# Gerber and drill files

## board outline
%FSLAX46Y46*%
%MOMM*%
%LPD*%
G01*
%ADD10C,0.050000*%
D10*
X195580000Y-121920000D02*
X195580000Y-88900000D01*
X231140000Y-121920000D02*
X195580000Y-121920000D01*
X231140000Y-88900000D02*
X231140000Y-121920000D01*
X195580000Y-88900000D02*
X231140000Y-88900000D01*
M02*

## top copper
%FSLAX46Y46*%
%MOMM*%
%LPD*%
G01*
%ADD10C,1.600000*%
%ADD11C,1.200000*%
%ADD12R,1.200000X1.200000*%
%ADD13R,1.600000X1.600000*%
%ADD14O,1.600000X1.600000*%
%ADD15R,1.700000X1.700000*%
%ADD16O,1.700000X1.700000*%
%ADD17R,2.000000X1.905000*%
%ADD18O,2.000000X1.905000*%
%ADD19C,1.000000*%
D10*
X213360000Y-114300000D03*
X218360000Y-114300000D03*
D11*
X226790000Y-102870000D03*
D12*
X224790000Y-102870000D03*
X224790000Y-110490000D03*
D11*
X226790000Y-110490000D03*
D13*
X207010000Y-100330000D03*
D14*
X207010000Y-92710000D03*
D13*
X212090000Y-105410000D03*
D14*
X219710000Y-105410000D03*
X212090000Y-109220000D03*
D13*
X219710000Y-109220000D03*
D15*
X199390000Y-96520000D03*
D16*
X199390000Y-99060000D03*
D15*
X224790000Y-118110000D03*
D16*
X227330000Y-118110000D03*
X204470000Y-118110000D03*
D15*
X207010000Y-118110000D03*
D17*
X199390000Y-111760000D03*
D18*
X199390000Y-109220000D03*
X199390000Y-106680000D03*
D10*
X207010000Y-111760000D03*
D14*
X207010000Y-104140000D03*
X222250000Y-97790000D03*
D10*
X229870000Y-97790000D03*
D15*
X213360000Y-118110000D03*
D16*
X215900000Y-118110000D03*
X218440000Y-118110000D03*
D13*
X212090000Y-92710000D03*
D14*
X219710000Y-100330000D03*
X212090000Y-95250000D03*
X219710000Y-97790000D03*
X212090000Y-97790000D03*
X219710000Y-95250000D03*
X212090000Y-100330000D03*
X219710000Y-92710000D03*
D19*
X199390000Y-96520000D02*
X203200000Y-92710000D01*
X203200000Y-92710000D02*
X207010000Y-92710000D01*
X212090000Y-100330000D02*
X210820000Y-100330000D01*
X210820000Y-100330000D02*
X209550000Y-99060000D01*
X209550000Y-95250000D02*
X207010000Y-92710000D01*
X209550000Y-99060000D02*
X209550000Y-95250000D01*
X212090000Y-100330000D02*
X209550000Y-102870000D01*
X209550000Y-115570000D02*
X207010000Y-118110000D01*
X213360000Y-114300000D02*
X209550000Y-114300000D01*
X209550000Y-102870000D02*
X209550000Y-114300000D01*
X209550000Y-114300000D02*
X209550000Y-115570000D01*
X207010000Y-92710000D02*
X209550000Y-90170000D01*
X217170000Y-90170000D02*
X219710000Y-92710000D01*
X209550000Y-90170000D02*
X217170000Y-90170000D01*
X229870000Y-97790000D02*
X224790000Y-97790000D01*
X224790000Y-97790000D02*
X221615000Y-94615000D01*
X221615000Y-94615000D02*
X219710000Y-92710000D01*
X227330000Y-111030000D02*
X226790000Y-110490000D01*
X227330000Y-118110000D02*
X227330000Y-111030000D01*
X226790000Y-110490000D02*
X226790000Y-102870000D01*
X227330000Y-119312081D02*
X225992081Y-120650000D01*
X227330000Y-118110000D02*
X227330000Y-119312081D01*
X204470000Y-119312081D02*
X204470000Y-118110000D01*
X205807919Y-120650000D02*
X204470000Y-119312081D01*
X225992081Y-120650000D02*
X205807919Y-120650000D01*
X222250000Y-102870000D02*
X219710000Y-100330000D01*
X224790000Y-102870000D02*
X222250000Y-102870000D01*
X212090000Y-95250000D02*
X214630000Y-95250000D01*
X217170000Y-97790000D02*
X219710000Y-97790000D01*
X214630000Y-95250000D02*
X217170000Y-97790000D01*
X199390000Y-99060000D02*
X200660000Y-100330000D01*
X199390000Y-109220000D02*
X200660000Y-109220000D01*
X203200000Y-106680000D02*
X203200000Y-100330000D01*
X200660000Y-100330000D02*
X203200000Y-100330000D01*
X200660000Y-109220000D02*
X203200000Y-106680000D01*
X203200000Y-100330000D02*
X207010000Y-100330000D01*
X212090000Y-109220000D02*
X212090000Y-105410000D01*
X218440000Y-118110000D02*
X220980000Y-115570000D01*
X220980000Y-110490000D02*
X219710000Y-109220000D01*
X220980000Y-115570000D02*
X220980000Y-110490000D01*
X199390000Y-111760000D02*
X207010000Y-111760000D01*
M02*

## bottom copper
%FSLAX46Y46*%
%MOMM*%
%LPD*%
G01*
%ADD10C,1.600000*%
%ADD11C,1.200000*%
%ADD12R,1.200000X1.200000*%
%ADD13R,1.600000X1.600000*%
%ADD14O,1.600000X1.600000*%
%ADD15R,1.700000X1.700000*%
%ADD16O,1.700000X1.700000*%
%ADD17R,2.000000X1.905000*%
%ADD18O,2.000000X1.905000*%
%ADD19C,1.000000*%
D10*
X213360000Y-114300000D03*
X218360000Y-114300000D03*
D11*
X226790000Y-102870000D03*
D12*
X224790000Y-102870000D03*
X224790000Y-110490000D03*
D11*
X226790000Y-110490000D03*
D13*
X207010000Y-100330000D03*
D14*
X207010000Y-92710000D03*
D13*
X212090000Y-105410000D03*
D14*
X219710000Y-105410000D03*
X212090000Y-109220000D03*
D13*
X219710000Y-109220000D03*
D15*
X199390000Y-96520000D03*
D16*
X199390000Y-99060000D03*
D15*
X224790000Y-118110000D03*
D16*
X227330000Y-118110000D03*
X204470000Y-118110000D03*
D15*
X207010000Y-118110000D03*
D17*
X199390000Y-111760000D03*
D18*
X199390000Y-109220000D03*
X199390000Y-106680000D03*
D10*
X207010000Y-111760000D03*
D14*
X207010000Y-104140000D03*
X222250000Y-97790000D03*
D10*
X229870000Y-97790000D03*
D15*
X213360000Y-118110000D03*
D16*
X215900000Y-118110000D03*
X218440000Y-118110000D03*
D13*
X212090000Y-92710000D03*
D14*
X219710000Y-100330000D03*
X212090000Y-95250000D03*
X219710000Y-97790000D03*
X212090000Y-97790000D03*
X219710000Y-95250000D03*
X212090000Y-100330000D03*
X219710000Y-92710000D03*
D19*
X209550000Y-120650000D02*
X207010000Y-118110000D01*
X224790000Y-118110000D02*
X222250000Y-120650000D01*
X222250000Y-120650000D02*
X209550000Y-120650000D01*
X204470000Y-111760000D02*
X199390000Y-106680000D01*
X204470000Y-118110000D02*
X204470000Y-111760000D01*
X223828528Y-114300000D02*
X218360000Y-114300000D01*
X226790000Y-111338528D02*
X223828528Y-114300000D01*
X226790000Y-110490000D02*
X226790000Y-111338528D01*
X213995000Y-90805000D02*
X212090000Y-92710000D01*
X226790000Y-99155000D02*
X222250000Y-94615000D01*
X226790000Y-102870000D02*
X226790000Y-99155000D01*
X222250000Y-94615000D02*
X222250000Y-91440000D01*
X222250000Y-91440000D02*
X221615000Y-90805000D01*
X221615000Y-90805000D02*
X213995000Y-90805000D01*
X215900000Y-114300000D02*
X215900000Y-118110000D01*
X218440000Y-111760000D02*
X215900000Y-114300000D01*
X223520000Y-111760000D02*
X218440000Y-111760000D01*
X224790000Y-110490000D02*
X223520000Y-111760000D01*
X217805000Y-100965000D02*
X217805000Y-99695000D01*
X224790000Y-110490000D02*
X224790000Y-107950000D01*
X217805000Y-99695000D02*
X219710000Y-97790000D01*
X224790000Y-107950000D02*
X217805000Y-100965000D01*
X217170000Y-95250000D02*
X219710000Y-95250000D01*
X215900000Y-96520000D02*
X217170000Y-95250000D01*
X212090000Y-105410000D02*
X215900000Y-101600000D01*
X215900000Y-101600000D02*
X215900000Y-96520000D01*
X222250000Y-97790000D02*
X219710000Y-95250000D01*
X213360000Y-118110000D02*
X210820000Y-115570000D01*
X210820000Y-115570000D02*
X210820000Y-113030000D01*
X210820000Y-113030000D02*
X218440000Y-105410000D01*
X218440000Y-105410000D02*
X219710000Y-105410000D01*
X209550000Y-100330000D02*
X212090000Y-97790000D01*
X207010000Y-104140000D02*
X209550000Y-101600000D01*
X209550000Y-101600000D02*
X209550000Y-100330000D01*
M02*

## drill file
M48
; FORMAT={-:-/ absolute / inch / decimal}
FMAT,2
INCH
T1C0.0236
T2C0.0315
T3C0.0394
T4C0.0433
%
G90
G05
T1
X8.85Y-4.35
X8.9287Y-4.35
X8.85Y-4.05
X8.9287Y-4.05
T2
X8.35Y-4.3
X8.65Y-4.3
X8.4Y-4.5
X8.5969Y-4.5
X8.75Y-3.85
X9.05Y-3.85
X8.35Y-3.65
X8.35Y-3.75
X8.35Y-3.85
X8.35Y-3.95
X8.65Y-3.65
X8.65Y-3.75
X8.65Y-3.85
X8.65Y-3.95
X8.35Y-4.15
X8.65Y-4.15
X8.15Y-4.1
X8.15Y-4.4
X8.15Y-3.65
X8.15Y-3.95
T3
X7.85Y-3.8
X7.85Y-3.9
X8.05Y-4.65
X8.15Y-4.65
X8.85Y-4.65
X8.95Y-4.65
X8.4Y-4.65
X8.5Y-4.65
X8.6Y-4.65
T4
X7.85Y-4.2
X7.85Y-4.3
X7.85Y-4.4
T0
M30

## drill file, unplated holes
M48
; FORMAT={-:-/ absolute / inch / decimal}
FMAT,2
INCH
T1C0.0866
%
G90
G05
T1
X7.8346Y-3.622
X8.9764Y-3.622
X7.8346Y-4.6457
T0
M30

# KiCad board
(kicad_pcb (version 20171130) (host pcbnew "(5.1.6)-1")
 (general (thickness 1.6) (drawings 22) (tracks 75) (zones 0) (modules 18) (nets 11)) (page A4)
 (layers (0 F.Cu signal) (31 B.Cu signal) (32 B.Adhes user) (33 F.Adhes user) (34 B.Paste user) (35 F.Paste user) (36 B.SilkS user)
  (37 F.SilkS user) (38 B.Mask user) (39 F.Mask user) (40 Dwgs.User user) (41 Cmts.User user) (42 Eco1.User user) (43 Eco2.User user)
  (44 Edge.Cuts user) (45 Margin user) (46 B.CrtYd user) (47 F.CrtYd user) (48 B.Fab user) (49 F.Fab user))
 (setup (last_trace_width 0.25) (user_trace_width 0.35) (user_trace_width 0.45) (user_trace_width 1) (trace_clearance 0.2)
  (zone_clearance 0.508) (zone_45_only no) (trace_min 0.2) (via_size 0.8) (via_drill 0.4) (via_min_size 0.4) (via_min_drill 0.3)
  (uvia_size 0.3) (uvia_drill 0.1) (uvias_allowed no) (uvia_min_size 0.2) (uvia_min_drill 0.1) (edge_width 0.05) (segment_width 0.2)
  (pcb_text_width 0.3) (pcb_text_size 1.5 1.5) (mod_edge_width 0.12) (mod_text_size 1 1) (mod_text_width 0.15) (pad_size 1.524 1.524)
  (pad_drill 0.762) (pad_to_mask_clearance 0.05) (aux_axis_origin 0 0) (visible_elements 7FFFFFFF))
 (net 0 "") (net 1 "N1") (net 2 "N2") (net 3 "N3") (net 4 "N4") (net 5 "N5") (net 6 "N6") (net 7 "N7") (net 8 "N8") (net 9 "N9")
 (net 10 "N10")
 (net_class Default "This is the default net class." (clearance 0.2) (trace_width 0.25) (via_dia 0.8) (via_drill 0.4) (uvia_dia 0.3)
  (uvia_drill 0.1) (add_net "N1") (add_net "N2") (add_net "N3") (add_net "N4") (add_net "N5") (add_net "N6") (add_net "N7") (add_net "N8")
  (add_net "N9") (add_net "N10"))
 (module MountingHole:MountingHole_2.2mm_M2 (layer F.Cu) (at 199 118)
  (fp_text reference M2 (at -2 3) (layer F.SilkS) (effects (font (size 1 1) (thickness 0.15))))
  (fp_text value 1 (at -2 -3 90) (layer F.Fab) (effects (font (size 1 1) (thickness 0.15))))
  (pad 1 np_thru_hole circle (at 0 0) (size 2.2 2.2) (drill 2.2) (layers *.Cu *.Mask)))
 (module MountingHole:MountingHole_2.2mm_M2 (layer F.Cu) (at 228 92)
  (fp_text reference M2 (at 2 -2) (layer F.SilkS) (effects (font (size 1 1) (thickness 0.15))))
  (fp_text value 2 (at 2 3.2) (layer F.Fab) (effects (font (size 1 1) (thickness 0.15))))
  (pad 1 np_thru_hole circle (at 0 0) (size 2.2 2.2) (drill 2.2) (layers *.Cu *.Mask)))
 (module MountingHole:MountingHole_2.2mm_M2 (layer F.Cu) (at 199 92)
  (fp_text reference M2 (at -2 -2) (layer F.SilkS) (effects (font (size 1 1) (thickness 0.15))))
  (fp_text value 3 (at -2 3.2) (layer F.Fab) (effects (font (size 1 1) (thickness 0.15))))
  (pad 1 np_thru_hole circle (at 0 0) (size 2.2 2.2) (drill 2.2) (layers *.Cu *.Mask)))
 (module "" (layer F.Cu) (at 133.35 157.48)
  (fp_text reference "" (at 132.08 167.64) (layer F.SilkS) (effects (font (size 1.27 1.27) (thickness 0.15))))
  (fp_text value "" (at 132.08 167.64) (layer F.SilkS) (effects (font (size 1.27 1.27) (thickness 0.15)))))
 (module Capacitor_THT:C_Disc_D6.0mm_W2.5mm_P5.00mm (layer F.Cu) (at 213.36 114.3)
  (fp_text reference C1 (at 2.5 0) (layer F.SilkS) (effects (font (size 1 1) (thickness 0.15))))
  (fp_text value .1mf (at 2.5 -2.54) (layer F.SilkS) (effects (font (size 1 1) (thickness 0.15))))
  (pad 1 thru_hole circle (at 0 0) (size 1.6 1.6) (drill 0.8) (layers *.Cu *.Mask) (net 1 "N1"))
  (pad 2 thru_hole circle (at 5 0) (size 1.6 1.6) (drill 0.8) (layers *.Cu *.Mask) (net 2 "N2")))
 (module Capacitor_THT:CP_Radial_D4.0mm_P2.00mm (layer F.Cu) (at 224.79 102.87)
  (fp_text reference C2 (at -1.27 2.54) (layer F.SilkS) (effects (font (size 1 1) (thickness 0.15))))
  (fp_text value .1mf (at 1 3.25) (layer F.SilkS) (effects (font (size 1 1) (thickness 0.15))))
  (pad 2 thru_hole circle (at 2 0) (size 1.2 1.2) (drill 0.6) (layers *.Cu *.Mask) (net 2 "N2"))
  (pad 1 thru_hole rect (at 0 0) (size 1.2 1.2) (drill 0.6) (layers *.Cu *.Mask) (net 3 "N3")))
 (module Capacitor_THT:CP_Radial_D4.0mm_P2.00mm (layer F.Cu) (at 224.79 110.49)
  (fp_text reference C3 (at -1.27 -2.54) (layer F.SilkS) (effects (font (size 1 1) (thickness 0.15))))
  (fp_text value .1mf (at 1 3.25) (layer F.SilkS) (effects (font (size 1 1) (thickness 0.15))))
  (pad 1 thru_hole rect (at 0 0) (size 1.2 1.2) (drill 0.6) (layers *.Cu *.Mask) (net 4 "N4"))
  (pad 2 thru_hole circle (at 2 0) (size 1.2 1.2) (drill 0.6) (layers *.Cu *.Mask) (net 2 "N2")))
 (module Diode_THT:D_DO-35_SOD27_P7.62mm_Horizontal (layer F.Cu) (at 207.01 100.33 90)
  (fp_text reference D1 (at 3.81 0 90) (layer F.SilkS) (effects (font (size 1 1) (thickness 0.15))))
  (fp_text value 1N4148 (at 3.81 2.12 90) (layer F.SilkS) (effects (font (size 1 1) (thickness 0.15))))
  (pad 1 thru_hole rect (at 0 0 90) (size 1.6 1.6) (drill 0.8) (layers *.Cu *.Mask) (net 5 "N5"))
  (pad 2 thru_hole oval (at 7.62 0 90) (size 1.6 1.6) (drill 0.8) (layers *.Cu *.Mask) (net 1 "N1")))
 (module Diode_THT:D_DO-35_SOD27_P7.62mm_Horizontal (layer F.Cu) (at 212.09 105.41)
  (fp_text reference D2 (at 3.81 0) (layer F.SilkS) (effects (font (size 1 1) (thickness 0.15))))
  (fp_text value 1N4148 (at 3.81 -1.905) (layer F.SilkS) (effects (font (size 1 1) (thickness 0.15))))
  (pad 1 thru_hole rect (at 0 0) (size 1.6 1.6) (drill 0.8) (layers *.Cu *.Mask) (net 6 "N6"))
  (pad 2 thru_hole oval (at 7.62 0) (size 1.6 1.6) (drill 0.8) (layers *.Cu *.Mask) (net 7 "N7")))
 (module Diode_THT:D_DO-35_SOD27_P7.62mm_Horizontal (layer F.Cu) (at 219.71 109.22 180)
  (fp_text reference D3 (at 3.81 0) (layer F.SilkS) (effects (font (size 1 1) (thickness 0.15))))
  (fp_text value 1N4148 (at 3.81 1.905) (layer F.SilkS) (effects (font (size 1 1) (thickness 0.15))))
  (pad 2 thru_hole oval (at 7.62 0 180) (size 1.6 1.6) (drill 0.8) (layers *.Cu *.Mask) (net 6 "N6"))
  (pad 1 thru_hole rect (at 0 0 180) (size 1.6 1.6) (drill 0.8) (layers *.Cu *.Mask) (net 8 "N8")))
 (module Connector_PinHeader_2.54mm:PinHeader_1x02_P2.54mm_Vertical (layer F.Cu) (at 199.39 96.52)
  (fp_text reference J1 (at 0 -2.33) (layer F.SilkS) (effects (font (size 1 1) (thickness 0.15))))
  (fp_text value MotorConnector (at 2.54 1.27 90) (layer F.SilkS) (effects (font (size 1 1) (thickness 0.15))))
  (pad 1 thru_hole rect (at 0 0) (size 1.7 1.7) (drill 1) (layers *.Cu *.Mask) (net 1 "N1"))
  (pad 2 thru_hole oval (at 0 2.54) (size 1.7 1.7) (drill 1) (layers *.Cu *.Mask) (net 5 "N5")))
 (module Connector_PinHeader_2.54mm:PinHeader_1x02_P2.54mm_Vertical (layer F.Cu) (at 224.79 118.11 90)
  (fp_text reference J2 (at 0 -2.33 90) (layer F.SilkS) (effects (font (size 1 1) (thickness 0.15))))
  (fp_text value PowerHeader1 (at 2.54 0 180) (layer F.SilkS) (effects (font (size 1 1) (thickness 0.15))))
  (pad 1 thru_hole rect (at 0 0 90) (size 1.7 1.7) (drill 1) (layers *.Cu *.Mask) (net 1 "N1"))
  (pad 2 thru_hole oval (at 0 2.54 90) (size 1.7 1.7) (drill 1) (layers *.Cu *.Mask) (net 2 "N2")))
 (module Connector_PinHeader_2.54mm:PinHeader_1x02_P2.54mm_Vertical (layer F.Cu) (at 207.01 118.11 270)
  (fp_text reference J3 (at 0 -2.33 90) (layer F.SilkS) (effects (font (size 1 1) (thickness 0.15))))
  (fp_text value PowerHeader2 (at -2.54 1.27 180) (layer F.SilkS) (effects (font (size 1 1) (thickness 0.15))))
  (pad 2 thru_hole oval (at 0 2.54 270) (size 1.7 1.7) (drill 1) (layers *.Cu *.Mask) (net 2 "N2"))
  (pad 1 thru_hole rect (at 0 0 270) (size 1.7 1.7) (drill 1) (layers *.Cu *.Mask) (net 1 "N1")))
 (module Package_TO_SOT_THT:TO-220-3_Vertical (layer F.Cu) (at 199.39 111.76 90)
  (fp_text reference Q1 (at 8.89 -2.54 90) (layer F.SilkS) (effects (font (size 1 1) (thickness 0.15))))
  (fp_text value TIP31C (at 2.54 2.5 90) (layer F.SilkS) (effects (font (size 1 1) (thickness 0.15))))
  (pad 1 thru_hole rect (at 0 0 90) (size 1.905 2) (drill 1.1) (layers *.Cu *.Mask) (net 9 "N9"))
  (pad 2 thru_hole oval (at 2.54 0 90) (size 1.905 2) (drill 1.1) (layers *.Cu *.Mask) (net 5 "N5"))
  (pad 3 thru_hole oval (at 5.08 0 90) (size 1.905 2) (drill 1.1) (layers *.Cu *.Mask) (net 2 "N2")))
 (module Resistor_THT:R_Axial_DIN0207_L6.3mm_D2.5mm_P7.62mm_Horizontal (layer F.Cu) (at 207.01 111.76 90)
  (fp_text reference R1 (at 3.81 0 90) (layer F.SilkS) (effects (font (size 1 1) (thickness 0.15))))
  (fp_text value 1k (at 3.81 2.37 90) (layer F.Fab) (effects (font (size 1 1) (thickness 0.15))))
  (pad 1 thru_hole circle (at 0 0 90) (size 1.6 1.6) (drill 0.8) (layers *.Cu *.Mask) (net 9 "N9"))
  (pad 2 thru_hole oval (at 7.62 0 90) (size 1.6 1.6) (drill 0.8) (layers *.Cu *.Mask) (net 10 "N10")))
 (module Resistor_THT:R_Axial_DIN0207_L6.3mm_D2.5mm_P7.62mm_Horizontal (layer F.Cu) (at 229.87 97.79 180)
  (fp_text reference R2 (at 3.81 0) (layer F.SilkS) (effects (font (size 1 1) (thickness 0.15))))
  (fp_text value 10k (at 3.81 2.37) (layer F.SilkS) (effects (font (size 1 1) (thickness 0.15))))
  (pad 2 thru_hole oval (at 7.62 0 180) (size 1.6 1.6) (drill 0.8) (layers *.Cu *.Mask) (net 6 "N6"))
  (pad 1 thru_hole circle (at 0 0 180) (size 1.6 1.6) (drill 0.8) (layers *.Cu *.Mask) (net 1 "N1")))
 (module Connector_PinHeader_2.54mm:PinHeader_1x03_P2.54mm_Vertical (layer F.Cu) (at 213.36 118.11 90)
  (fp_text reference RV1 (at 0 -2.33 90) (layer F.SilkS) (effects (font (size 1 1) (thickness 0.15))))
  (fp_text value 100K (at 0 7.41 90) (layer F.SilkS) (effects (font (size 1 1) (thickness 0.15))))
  (pad 1 thru_hole rect (at 0 0 90) (size 1.7 1.7) (drill 1) (layers *.Cu *.Mask) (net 7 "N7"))
  (pad 2 thru_hole oval (at 0 2.54 90) (size 1.7 1.7) (drill 1) (layers *.Cu *.Mask) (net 4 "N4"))
  (pad 3 thru_hole oval (at 0 5.08 90) (size 1.7 1.7) (drill 1) (layers *.Cu *.Mask) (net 8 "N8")))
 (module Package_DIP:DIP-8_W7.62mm (layer F.Cu) (at 212.09 92.71)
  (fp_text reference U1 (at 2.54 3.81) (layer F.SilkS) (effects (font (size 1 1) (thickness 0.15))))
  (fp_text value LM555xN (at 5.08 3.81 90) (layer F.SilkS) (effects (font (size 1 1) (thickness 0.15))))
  (pad 1 thru_hole rect (at 0 0) (size 1.6 1.6) (drill 0.8) (layers *.Cu *.Mask) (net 2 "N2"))
  (pad 5 thru_hole oval (at 7.62 7.62) (size 1.6 1.6) (drill 0.8) (layers *.Cu *.Mask) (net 3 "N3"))
  (pad 2 thru_hole oval (at 0 2.54) (size 1.6 1.6) (drill 0.8) (layers *.Cu *.Mask) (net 4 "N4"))
  (pad 6 thru_hole oval (at 7.62 5.08) (size 1.6 1.6) (drill 0.8) (layers *.Cu *.Mask) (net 4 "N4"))
  (pad 3 thru_hole oval (at 0 5.08) (size 1.6 1.6) (drill 0.8) (layers *.Cu *.Mask) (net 10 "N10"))
  (pad 7 thru_hole oval (at 7.62 2.54) (size 1.6 1.6) (drill 0.8) (layers *.Cu *.Mask) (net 6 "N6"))
  (pad 4 thru_hole oval (at 0 7.62) (size 1.6 1.6) (drill 0.8) (layers *.Cu *.Mask) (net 1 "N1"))
  (pad 8 thru_hole oval (at 7.62 0) (size 1.6 1.6) (drill 0.8) (layers *.Cu *.Mask) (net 1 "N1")))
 (gr_line (start 195.58 121.92) (end 195.58 88.9) (layer Edge.Cuts) (width 0.05))
 (gr_line (start 231.14 121.92) (end 195.58 121.92) (layer Edge.Cuts) (width 0.05))
 (gr_line (start 231.14 88.9) (end 231.14 121.92) (layer Edge.Cuts) (width 0.05))
 (gr_line (start 195.58 88.9) (end 231.14 88.9) (layer Edge.Cuts) (width 0.05))
 (segment (start 199.39 96.52) (end 203.2 92.71) (width 1) (layer F.Cu) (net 1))
 (segment (start 203.2 92.71) (end 207.01 92.71) (width 1) (layer F.Cu) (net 1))
 (segment (start 212.09 100.33) (end 210.82 100.33) (width 1) (layer F.Cu) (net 1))
 (segment (start 210.82 100.33) (end 209.55 99.06) (width 1) (layer F.Cu) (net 1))
 (segment (start 209.55 95.25) (end 207.01 92.71) (width 1) (layer F.Cu) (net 1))
 (segment (start 209.55 99.06) (end 209.55 95.25) (width 1) (layer F.Cu) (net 1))
 (segment (start 212.09 100.33) (end 209.55 102.87) (width 1) (layer F.Cu) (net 1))
 (segment (start 209.55 115.57) (end 207.01 118.11) (width 1) (layer F.Cu) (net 1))
 (segment (start 213.36 114.3) (end 209.55 114.3) (width 1) (layer F.Cu) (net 1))
 (segment (start 209.55 102.87) (end 209.55 114.3) (width 1) (layer F.Cu) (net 1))
 (segment (start 209.55 114.3) (end 209.55 115.57) (width 1) (layer F.Cu) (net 1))
 (segment (start 207.01 92.71) (end 209.55 90.17) (width 1) (layer F.Cu) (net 1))
 (segment (start 217.17 90.17) (end 219.71 92.71) (width 1) (layer F.Cu) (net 1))
 (segment (start 209.55 90.17) (end 217.17 90.17) (width 1) (layer F.Cu) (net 1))
 (segment (start 209.55 120.65) (end 207.01 118.11) (width 1) (layer B.Cu) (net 1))
 (segment (start 224.79 118.11) (end 222.25 120.65) (width 1) (layer B.Cu) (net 1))
 (segment (start 222.25 120.65) (end 209.55 120.65) (width 1) (layer B.Cu) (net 1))
 (segment (start 229.87 97.79) (end 224.79 97.79) (width 1) (layer F.Cu) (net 1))
 (segment (start 224.79 97.79) (end 221.615 94.615) (width 1) (layer F.Cu) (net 1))
 (segment (start 221.615 94.615) (end 219.71 92.71) (width 1) (layer F.Cu) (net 1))
 (segment (start 227.33 111.03) (end 226.79 110.49) (width 1) (layer F.Cu) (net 2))
 (segment (start 227.33 118.11) (end 227.33 111.03) (width 1) (layer F.Cu) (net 2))
 (segment (start 226.79 110.49) (end 226.79 102.87) (width 1) (layer F.Cu) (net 2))
 (segment (start 204.47 111.76) (end 199.39 106.68) (width 1) (layer B.Cu) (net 2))
 (segment (start 204.47 118.11) (end 204.47 111.76) (width 1) (layer B.Cu) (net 2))
 (segment (start 223.828528 114.3) (end 218.36 114.3) (width 1) (layer B.Cu) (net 2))
 (segment (start 226.79 111.338528) (end 223.828528 114.3) (width 1) (layer B.Cu) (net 2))
 (segment (start 226.79 110.49) (end 226.79 111.338528) (width 1) (layer B.Cu) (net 2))
 (segment (start 227.33 119.312081) (end 225.992081 120.65) (width 1) (layer F.Cu) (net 2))
 (segment (start 227.33 118.11) (end 227.33 119.312081) (width 1) (layer F.Cu) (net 2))
 (segment (start 204.47 119.312081) (end 204.47 118.11) (width 1) (layer F.Cu) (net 2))
 (segment (start 205.807919 120.65) (end 204.47 119.312081) (width 1) (layer F.Cu) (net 2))
 (segment (start 225.992081 120.65) (end 205.807919 120.65) (width 1) (layer F.Cu) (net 2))
 (segment (start 213.995 90.805) (end 212.09 92.71) (width 1) (layer B.Cu) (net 2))
 (segment (start 226.79 99.155) (end 222.25 94.615) (width 1) (layer B.Cu) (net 2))
 (segment (start 226.79 102.87) (end 226.79 99.155) (width 1) (layer B.Cu) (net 2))
 (segment (start 222.25 94.615) (end 222.25 91.44) (width 1) (layer B.Cu) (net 2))
 (segment (start 222.25 91.44) (end 221.615 90.805) (width 1) (layer B.Cu) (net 2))
 (segment (start 221.615 90.805) (end 213.995 90.805) (width 1) (layer B.Cu) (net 2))
 (segment (start 222.25 102.87) (end 219.71 100.33) (width 1) (layer F.Cu) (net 3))
 (segment (start 224.79 102.87) (end 222.25 102.87) (width 1) (layer F.Cu) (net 3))
 (segment (start 212.09 95.25) (end 214.63 95.25) (width 1) (layer F.Cu) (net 4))
 (segment (start 217.17 97.79) (end 219.71 97.79) (width 1) (layer F.Cu) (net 4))
 (segment (start 214.63 95.25) (end 217.17 97.79) (width 1) (layer F.Cu) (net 4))
 (segment (start 215.9 114.3) (end 215.9 118.11) (width 1) (layer B.Cu) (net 4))
 (segment (start 218.44 111.76) (end 215.9 114.3) (width 1) (layer B.Cu) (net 4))
 (segment (start 223.52 111.76) (end 218.44 111.76) (width 1) (layer B.Cu) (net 4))
 (segment (start 224.79 110.49) (end 223.52 111.76) (width 1) (layer B.Cu) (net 4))
 (segment (start 217.805 100.965) (end 217.805 99.695) (width 1) (layer B.Cu) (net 4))
 (segment (start 224.79 110.49) (end 224.79 107.95) (width 1) (layer B.Cu) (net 4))
 (segment (start 217.805 99.695) (end 219.71 97.79) (width 1) (layer B.Cu) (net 4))
 (segment (start 224.79 107.95) (end 217.805 100.965) (width 1) (layer B.Cu) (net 4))
 (segment (start 199.39 99.06) (end 200.66 100.33) (width 1) (layer F.Cu) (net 5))
 (segment (start 199.39 109.22) (end 200.66 109.22) (width 1) (layer F.Cu) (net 5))
 (segment (start 203.2 106.68) (end 203.2 100.33) (width 1) (layer F.Cu) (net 5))
 (segment (start 200.66 100.33) (end 203.2 100.33) (width 1) (layer F.Cu) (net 5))
 (segment (start 200.66 109.22) (end 203.2 106.68) (width 1) (layer F.Cu) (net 5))
 (segment (start 203.2 100.33) (end 207.01 100.33) (width 1) (layer F.Cu) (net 5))
 (segment (start 212.09 109.22) (end 212.09 105.41) (width 1) (layer F.Cu) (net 6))
 (segment (start 217.17 95.25) (end 219.71 95.25) (width 1) (layer B.Cu) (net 6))
 (segment (start 215.9 96.52) (end 217.17 95.25) (width 1) (layer B.Cu) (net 6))
 (segment (start 212.09 105.41) (end 215.9 101.6) (width 1) (layer B.Cu) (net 6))
 (segment (start 215.9 101.6) (end 215.9 96.52) (width 1) (layer B.Cu) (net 6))
 (segment (start 222.25 97.79) (end 219.71 95.25) (width 1) (layer B.Cu) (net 6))
 (segment (start 213.36 118.11) (end 210.82 115.57) (width 1) (layer B.Cu) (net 7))
 (segment (start 210.82 115.57) (end 210.82 113.03) (width 1) (layer B.Cu) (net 7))
 (segment (start 210.82 113.03) (end 218.44 105.41) (width 1) (layer B.Cu) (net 7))
 (segment (start 218.44 105.41) (end 219.71 105.41) (width 1) (layer B.Cu) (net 7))
 (segment (start 218.44 118.11) (end 220.98 115.57) (width 1) (layer F.Cu) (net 8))
 (segment (start 220.98 110.49) (end 219.71 109.22) (width 1) (layer F.Cu) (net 8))
 (segment (start 220.98 115.57) (end 220.98 110.49) (width 1) (layer F.Cu) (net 8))
 (segment (start 199.39 111.76) (end 207.01 111.76) (width 1) (layer F.Cu) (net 9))
 (segment (start 209.55 100.33) (end 212.09 97.79) (width 1) (layer B.Cu) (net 10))
 (segment (start 207.01 104.14) (end 209.55 101.6) (width 1) (layer B.Cu) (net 10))
 (segment (start 209.55 101.6) (end 209.55 100.33) (width 1) (layer B.Cu) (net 10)))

